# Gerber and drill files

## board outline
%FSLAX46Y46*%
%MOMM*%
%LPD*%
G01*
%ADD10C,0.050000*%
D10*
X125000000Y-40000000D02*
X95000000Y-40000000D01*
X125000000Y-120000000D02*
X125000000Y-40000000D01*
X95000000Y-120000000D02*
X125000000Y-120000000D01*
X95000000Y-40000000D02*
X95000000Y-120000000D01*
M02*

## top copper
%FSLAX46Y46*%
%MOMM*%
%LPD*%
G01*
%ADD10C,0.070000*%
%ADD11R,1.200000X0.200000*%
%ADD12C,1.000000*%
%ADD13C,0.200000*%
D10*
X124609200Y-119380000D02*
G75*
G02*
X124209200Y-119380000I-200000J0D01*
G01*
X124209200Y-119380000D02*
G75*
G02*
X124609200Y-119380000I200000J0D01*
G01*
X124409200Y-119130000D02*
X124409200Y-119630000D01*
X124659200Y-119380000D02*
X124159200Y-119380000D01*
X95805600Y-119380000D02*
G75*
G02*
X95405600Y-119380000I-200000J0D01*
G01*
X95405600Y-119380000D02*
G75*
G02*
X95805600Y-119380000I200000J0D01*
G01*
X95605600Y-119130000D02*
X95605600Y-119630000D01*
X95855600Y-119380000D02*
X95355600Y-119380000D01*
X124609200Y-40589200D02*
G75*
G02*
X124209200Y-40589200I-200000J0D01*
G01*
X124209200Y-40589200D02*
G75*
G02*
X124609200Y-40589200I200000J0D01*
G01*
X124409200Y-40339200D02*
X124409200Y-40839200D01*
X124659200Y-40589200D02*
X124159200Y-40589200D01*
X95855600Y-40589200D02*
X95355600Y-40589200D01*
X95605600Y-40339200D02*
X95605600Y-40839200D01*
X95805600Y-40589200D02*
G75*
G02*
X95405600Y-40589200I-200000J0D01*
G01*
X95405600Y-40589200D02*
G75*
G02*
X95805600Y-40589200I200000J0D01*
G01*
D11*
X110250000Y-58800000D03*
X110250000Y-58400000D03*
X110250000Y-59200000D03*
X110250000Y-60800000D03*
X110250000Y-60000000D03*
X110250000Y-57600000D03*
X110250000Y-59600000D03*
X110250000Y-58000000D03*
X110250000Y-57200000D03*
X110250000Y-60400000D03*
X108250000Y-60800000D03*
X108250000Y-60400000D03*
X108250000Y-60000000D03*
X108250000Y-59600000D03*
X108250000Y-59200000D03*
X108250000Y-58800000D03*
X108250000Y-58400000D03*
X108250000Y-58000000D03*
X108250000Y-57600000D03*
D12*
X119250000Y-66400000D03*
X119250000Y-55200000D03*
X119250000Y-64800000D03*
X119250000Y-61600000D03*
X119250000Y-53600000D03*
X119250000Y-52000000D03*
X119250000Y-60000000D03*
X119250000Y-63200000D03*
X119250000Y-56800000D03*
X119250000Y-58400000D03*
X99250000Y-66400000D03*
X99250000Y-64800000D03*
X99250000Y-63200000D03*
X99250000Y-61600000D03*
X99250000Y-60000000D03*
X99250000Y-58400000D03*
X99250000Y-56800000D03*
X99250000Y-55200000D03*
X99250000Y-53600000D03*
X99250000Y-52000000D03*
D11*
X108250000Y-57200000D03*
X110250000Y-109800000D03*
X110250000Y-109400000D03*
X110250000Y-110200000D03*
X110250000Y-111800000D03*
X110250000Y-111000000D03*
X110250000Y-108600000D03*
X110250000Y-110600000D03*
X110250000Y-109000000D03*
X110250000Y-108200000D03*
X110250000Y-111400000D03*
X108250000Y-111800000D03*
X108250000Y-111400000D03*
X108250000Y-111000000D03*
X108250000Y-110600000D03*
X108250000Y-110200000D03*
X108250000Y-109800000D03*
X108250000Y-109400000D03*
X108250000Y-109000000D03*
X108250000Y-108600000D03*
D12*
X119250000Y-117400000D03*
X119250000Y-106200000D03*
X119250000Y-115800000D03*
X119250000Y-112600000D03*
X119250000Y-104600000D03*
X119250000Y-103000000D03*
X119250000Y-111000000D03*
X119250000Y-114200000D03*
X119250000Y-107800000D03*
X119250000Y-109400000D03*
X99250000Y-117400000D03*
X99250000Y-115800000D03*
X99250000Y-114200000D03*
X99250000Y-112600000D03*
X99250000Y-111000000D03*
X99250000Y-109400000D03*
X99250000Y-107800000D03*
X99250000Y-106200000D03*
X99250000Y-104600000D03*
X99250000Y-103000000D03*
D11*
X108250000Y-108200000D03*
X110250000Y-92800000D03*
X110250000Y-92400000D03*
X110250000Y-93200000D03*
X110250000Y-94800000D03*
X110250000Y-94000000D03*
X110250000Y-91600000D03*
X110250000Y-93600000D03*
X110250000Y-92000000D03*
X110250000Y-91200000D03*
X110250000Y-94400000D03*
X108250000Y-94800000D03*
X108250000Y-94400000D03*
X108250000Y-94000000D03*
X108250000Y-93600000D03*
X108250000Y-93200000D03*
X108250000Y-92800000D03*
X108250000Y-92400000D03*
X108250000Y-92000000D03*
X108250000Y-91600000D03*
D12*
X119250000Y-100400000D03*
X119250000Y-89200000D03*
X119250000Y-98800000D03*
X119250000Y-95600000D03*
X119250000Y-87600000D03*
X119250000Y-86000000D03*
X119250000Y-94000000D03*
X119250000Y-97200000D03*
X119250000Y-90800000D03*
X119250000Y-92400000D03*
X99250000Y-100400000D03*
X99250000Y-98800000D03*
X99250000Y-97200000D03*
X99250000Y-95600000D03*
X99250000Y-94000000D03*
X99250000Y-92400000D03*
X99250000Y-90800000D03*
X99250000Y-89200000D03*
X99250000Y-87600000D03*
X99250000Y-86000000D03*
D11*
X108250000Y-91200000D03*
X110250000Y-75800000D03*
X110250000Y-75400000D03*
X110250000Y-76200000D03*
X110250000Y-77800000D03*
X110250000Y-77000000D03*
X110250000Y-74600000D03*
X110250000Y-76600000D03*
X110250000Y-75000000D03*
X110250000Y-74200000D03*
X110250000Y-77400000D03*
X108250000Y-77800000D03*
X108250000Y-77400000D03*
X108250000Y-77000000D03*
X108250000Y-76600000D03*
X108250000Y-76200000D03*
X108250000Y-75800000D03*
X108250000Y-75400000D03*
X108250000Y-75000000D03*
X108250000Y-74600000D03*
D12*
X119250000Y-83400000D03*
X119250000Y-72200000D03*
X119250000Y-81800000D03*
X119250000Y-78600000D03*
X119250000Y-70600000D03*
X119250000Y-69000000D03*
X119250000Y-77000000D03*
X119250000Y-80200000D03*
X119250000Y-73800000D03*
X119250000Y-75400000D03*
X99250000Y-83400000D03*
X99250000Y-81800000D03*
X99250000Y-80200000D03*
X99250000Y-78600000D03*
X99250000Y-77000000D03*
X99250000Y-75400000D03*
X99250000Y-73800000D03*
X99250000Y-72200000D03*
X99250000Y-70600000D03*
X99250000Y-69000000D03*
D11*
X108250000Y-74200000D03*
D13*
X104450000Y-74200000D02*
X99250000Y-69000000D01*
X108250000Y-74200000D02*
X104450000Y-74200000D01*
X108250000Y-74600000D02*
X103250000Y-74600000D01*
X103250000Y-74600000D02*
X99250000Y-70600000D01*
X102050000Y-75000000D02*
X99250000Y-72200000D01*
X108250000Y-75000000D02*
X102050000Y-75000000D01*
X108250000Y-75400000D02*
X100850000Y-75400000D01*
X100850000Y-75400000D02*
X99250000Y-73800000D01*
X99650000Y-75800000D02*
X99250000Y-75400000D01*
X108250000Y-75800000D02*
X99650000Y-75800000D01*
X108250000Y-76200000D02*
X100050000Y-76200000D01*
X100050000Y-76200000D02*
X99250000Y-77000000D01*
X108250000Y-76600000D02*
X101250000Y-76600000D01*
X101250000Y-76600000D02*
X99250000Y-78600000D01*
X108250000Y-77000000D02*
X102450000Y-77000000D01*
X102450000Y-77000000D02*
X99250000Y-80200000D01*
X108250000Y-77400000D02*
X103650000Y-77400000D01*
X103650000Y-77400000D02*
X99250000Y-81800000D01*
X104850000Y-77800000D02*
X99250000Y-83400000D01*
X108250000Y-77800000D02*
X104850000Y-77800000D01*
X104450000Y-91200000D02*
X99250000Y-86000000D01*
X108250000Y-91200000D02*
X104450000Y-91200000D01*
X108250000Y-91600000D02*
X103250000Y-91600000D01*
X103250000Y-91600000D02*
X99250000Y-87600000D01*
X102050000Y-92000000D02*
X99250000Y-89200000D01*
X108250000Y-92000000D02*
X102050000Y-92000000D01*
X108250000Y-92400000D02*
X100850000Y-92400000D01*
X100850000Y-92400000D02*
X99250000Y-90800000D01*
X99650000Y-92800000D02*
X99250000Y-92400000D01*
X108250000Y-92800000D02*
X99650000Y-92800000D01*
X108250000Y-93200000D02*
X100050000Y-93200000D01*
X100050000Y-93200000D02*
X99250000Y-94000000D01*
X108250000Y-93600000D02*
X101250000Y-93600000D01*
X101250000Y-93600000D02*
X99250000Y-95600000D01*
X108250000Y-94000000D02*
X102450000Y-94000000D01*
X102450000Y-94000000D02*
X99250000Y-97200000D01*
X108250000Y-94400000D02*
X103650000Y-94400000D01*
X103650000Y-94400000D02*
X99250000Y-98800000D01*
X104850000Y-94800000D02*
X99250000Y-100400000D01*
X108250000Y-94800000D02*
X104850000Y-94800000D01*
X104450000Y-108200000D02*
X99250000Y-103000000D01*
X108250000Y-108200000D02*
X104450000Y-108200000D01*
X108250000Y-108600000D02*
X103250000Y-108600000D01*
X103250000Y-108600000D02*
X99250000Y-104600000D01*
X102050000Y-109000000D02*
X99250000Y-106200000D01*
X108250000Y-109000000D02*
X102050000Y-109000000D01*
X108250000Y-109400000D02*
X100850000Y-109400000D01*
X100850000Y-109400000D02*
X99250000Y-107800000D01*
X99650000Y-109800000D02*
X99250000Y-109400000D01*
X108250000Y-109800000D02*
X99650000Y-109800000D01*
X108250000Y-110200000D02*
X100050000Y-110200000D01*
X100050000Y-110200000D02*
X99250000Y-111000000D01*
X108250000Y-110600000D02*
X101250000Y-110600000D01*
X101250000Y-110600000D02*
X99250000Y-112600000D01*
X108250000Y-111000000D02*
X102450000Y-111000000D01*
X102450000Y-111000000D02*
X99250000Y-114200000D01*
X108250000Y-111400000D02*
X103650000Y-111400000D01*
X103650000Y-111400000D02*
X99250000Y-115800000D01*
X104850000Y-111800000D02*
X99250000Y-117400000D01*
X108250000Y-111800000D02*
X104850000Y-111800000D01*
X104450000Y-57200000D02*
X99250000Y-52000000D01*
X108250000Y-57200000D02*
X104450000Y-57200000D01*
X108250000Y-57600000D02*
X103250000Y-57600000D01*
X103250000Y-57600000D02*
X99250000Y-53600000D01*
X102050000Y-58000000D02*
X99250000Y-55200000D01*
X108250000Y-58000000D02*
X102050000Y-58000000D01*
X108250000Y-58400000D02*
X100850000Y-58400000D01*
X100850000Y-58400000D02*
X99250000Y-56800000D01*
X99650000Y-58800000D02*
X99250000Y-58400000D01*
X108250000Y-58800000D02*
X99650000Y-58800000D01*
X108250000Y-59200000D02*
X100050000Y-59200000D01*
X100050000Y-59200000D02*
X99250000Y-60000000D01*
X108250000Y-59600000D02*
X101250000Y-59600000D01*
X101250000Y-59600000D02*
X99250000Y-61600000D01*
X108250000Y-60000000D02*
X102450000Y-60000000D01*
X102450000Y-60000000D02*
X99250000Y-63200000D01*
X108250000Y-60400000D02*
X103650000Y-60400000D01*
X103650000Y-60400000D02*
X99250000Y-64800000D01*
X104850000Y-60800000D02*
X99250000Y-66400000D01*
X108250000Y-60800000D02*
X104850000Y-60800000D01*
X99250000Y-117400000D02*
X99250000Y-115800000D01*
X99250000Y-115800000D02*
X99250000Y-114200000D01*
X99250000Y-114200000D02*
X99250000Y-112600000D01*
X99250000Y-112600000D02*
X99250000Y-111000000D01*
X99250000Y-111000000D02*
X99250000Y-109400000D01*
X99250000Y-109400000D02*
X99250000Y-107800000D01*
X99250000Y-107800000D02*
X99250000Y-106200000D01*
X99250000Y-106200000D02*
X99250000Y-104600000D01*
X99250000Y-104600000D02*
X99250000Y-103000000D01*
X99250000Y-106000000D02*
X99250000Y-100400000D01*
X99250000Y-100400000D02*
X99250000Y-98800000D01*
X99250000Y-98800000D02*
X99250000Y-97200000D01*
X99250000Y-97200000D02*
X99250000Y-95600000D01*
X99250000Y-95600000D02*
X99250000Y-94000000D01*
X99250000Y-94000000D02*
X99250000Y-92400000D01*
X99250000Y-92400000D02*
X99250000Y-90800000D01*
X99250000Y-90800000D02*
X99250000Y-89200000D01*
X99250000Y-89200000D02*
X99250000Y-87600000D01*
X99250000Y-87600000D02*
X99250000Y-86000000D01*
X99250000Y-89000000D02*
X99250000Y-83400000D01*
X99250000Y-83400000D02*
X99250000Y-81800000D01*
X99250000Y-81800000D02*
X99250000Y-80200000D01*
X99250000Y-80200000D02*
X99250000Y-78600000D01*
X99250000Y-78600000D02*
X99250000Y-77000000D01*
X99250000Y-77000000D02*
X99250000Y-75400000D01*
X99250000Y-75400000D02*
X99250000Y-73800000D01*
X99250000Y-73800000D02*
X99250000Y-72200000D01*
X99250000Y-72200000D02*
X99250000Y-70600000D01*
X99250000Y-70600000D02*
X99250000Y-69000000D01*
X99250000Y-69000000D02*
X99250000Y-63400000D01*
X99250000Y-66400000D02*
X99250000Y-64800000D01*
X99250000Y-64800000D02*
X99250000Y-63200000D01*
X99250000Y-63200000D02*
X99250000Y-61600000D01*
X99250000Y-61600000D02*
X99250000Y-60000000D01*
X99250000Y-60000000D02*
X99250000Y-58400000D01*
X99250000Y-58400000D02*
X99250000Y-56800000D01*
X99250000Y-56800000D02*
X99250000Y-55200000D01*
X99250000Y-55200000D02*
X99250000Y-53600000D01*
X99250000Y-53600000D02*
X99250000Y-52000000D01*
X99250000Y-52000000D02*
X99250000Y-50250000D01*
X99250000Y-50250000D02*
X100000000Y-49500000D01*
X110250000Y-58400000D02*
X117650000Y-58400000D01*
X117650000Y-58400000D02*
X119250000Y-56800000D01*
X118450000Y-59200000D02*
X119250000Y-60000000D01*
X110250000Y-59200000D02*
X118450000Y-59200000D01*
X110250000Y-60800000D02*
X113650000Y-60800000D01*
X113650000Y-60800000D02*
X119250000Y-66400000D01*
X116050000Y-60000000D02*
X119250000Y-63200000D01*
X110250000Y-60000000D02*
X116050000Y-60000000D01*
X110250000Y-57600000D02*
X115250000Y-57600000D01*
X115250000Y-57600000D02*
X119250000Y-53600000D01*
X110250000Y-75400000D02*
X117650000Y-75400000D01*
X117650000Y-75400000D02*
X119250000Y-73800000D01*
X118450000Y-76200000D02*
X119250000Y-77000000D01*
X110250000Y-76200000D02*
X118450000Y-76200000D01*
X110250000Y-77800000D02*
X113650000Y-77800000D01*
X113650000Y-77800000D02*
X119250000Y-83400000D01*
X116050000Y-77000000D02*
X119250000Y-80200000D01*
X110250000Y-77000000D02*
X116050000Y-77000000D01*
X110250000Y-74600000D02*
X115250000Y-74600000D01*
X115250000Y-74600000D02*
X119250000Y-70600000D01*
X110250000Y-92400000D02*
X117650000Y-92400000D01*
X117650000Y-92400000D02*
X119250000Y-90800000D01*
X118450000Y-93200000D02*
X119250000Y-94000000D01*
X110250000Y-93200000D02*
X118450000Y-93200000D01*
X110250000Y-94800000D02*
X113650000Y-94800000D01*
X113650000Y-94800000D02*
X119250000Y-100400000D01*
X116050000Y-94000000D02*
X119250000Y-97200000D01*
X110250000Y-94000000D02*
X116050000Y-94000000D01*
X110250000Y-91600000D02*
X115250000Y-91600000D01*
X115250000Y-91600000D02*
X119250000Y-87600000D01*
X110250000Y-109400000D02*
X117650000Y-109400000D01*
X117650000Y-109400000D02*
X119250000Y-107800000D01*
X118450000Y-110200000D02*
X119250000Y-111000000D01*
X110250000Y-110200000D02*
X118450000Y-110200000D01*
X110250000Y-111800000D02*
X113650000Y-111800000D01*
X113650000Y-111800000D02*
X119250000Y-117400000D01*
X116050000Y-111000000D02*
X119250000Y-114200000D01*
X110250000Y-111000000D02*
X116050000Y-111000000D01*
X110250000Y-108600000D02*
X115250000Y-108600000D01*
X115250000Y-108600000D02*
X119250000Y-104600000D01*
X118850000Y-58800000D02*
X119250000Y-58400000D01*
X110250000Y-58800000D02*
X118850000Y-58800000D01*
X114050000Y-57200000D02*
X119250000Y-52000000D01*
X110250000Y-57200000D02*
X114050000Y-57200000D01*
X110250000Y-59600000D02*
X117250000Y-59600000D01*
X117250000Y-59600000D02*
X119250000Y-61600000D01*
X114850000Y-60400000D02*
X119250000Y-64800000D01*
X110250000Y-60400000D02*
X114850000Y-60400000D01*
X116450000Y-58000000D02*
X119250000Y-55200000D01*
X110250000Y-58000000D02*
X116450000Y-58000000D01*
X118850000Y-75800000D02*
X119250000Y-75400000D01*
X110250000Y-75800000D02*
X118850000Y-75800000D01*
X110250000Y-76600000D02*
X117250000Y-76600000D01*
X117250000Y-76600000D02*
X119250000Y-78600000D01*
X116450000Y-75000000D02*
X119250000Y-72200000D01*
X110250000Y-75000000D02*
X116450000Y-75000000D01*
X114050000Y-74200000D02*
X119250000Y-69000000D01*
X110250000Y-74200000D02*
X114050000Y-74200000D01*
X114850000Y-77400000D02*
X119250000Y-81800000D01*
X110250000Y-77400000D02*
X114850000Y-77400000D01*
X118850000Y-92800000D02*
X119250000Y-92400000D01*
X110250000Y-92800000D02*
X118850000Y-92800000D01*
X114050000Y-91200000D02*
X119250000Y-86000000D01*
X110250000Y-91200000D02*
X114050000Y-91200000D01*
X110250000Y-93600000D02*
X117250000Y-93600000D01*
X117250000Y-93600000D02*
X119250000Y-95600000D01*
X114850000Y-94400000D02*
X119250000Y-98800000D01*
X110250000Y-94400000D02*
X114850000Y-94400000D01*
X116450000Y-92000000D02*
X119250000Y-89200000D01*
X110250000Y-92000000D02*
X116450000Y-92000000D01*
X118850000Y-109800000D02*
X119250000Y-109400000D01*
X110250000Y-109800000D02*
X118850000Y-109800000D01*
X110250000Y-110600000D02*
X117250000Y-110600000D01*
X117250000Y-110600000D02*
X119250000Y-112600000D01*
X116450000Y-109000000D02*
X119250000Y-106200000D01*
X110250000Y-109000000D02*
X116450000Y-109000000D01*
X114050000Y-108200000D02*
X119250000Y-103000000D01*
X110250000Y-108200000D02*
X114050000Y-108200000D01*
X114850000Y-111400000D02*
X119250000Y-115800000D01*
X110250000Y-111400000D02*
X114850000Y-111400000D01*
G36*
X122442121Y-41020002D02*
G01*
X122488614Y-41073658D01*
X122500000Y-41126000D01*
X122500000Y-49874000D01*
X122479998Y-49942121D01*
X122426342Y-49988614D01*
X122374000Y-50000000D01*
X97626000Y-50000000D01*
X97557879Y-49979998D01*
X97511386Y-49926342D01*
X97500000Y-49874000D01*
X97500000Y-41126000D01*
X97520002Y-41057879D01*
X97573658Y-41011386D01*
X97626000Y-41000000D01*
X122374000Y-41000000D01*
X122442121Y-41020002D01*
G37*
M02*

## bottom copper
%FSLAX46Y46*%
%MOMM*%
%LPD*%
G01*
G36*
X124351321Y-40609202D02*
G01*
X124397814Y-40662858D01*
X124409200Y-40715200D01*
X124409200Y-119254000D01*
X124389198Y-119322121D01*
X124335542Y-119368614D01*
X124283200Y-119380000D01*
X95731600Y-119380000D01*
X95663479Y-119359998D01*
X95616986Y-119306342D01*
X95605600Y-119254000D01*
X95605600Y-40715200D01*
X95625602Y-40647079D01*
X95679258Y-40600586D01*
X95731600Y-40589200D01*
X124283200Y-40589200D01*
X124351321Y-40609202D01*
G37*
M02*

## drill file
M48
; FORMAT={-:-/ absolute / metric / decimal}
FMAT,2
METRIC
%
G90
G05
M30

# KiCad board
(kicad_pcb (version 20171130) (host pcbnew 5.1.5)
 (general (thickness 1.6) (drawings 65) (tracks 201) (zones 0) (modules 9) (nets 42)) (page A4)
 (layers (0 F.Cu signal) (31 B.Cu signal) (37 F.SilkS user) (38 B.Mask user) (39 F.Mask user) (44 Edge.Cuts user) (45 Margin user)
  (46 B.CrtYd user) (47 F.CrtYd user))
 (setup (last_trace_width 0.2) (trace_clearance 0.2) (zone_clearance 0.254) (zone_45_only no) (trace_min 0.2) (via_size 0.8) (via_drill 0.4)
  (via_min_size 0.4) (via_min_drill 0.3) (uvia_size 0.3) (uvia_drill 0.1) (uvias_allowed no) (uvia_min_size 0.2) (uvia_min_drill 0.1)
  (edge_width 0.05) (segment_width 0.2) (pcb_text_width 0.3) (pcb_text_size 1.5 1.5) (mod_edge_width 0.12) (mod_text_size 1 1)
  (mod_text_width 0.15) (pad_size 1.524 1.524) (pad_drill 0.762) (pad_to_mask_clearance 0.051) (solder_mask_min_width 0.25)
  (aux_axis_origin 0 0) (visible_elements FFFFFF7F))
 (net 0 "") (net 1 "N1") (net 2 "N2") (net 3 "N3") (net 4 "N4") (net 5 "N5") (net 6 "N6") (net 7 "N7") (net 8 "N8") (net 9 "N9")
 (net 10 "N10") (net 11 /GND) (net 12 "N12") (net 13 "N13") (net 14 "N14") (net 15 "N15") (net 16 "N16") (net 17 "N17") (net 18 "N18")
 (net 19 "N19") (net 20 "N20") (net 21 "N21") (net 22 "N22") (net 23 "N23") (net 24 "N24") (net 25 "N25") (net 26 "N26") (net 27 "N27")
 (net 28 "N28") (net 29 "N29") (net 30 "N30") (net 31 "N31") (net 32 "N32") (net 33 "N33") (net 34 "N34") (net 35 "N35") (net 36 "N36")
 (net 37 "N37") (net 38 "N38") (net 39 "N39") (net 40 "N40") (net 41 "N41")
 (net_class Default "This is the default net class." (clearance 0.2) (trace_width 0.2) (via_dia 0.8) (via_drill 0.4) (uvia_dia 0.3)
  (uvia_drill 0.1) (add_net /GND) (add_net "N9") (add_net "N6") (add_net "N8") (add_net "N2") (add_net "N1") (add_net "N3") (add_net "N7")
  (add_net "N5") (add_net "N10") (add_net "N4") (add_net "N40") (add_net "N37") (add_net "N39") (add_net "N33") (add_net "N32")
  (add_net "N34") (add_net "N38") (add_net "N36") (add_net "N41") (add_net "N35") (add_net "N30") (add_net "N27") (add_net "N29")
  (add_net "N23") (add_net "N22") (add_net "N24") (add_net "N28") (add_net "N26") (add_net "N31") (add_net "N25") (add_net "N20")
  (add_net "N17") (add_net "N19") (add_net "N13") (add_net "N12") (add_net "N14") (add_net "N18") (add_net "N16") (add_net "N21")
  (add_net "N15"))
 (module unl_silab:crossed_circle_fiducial (layer F.Cu) (at 124.4092 119.38)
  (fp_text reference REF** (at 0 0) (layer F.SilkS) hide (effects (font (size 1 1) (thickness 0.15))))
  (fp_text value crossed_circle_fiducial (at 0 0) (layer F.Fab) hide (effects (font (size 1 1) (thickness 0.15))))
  (fp_circle (center 0 0) (end 0.2 0) (layer F.Cu) (width 0.07))
  (fp_line (start 0 -0.25) (end 0 0.25) (layer F.Cu) (width 0.07))
  (fp_line (start 0.25 0) (end -0.25 0) (layer F.Cu) (width 0.07)))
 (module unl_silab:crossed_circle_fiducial (layer F.Cu) (at 95.6056 119.38)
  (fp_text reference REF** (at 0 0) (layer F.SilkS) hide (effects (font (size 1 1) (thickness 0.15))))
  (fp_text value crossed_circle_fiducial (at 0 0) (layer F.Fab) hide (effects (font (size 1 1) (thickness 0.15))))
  (fp_circle (center 0 0) (end 0.2 0) (layer F.Cu) (width 0.07))
  (fp_line (start 0 -0.25) (end 0 0.25) (layer F.Cu) (width 0.07))
  (fp_line (start 0.25 0) (end -0.25 0) (layer F.Cu) (width 0.07)))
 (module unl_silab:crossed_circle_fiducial (layer F.Cu) (at 124.4092 40.5892)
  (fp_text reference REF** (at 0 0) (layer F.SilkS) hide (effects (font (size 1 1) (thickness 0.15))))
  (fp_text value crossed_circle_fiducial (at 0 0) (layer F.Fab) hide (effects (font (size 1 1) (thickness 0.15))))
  (fp_circle (center 0 0) (end 0.2 0) (layer F.Cu) (width 0.07))
  (fp_line (start 0 -0.25) (end 0 0.25) (layer F.Cu) (width 0.07))
  (fp_line (start 0.25 0) (end -0.25 0) (layer F.Cu) (width 0.07)))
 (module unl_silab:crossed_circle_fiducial (layer F.Cu) (at 95.6056 40.5892)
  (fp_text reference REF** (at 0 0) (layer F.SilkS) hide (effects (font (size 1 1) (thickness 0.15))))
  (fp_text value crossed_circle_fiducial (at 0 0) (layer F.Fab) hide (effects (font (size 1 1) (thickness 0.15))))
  (fp_line (start 0.25 0) (end -0.25 0) (layer F.Cu) (width 0.07))
  (fp_line (start 0 -0.25) (end 0 0.25) (layer F.Cu) (width 0.07))
  (fp_circle (center 0 0) (end 0.2 0) (layer F.Cu) (width 0.07)))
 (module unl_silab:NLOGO (layer F.Cu) (at 108.75 115.25)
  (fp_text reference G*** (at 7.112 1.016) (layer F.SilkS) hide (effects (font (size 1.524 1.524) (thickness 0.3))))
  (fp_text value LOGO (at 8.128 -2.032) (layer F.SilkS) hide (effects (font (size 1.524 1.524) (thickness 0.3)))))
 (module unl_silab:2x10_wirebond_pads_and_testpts (layer F.Cu) (at 109.25 59)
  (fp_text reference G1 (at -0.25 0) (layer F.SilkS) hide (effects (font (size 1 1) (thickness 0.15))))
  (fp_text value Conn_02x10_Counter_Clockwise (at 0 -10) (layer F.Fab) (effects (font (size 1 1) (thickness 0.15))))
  (pad 15 smd rect (at 1 -0.2) (size 1.2 0.2) (layers F.Cu F.Paste F.Mask) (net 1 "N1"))
  (pad 14 smd rect (at 1 -0.6) (size 1.2 0.2) (layers F.Cu F.Paste F.Mask) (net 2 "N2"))
  (pad 16 smd rect (at 1 0.2) (size 1.2 0.2) (layers F.Cu F.Paste F.Mask) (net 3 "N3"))
  (pad 20 smd rect (at 1 1.8) (size 1.2 0.2) (layers F.Cu F.Paste F.Mask) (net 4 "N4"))
  (pad 18 smd rect (at 1 1) (size 1.2 0.2) (layers F.Cu F.Paste F.Mask) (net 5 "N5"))
  (pad 12 smd rect (at 1 -1.4) (size 1.2 0.2) (layers F.Cu F.Paste F.Mask) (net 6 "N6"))
  (pad 17 smd rect (at 1 0.6) (size 1.2 0.2) (layers F.Cu F.Paste F.Mask) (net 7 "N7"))
  (pad 13 smd rect (at 1 -1) (size 1.2 0.2) (layers F.Cu F.Paste F.Mask) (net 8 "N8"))
  (pad 11 smd rect (at 1 -1.8) (size 1.2 0.2) (layers F.Cu F.Paste F.Mask) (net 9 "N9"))
  (pad 19 smd rect (at 1 1.4) (size 1.2 0.2) (layers F.Cu F.Paste F.Mask) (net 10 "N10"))
  (pad 10 smd rect (at -1 1.8) (size 1.2 0.2) (layers F.Cu F.Paste F.Mask) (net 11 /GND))
  (pad 9 smd rect (at -1 1.4) (size 1.2 0.2) (layers F.Cu F.Paste F.Mask) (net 11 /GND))
  (pad 8 smd rect (at -1 1) (size 1.2 0.2) (layers F.Cu F.Paste F.Mask) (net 11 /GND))
  (pad 7 smd rect (at -1 0.6) (size 1.2 0.2) (layers F.Cu F.Paste F.Mask) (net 11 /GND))
  (pad 6 smd rect (at -1 0.2) (size 1.2 0.2) (layers F.Cu F.Paste F.Mask) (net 11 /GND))
  (pad 5 smd rect (at -1 -0.2) (size 1.2 0.2) (layers F.Cu F.Paste F.Mask) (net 11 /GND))
  (pad 4 smd rect (at -1 -0.6) (size 1.2 0.2) (layers F.Cu F.Paste F.Mask) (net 11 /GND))
  (pad 3 smd rect (at -1 -1) (size 1.2 0.2) (layers F.Cu F.Paste F.Mask) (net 11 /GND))
  (pad 2 smd rect (at -1 -1.4) (size 1.2 0.2) (layers F.Cu F.Paste F.Mask) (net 11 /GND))
  (pad 20 smd circle (at 10 7.4) (size 1 1) (layers F.Cu F.Paste F.Mask) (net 4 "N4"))
  (pad 13 smd circle (at 10 -3.8) (size 1 1) (layers F.Cu F.Paste F.Mask) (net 8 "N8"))
  (pad 19 smd circle (at 10 5.8) (size 1 1) (layers F.Cu F.Paste F.Mask) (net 10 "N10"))
  (pad 17 smd circle (at 10 2.6) (size 1 1) (layers F.Cu F.Paste F.Mask) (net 7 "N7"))
  (pad 12 smd circle (at 10 -5.4) (size 1 1) (layers F.Cu F.Paste F.Mask) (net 6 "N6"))
  (pad 11 smd circle (at 10 -7) (size 1 1) (layers F.Cu F.Paste F.Mask) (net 9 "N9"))
  (pad 16 smd circle (at 10 1) (size 1 1) (layers F.Cu F.Paste F.Mask) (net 3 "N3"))
  (pad 18 smd circle (at 10 4.2) (size 1 1) (layers F.Cu F.Paste F.Mask) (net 5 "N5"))
  (pad 14 smd circle (at 10 -2.2) (size 1 1) (layers F.Cu F.Paste F.Mask) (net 2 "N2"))
  (pad 15 smd circle (at 10 -0.6) (size 1 1) (layers F.Cu F.Paste F.Mask) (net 1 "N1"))
  (pad 10 smd circle (at -10 7.4) (size 1 1) (layers F.Cu F.Paste F.Mask) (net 11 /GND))
  (pad 9 smd circle (at -10 5.8) (size 1 1) (layers F.Cu F.Paste F.Mask) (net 11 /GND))
  (pad 8 smd circle (at -10 4.2) (size 1 1) (layers F.Cu F.Paste F.Mask) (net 11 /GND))
  (pad 7 smd circle (at -10 2.6) (size 1 1) (layers F.Cu F.Paste F.Mask) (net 11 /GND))
  (pad 6 smd circle (at -10 1) (size 1 1) (layers F.Cu F.Paste F.Mask) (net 11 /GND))
  (pad 5 smd circle (at -10 -0.6) (size 1 1) (layers F.Cu F.Paste F.Mask) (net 11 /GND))
  (pad 4 smd circle (at -10 -2.2) (size 1 1) (layers F.Cu F.Paste F.Mask) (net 11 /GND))
  (pad 3 smd circle (at -10 -3.8) (size 1 1) (layers F.Cu F.Paste F.Mask) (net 11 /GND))
  (pad 2 smd circle (at -10 -5.4) (size 1 1) (layers F.Cu F.Paste F.Mask) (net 11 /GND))
  (pad 1 smd circle (at -10 -7) (size 1 1) (layers F.Cu F.Paste F.Mask) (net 11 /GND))
  (pad 1 smd rect (at -1 -1.8) (size 1.2 0.2) (layers F.Cu F.Paste F.Mask) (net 11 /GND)))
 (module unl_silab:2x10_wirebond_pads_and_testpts (layer F.Cu) (at 109.25 110)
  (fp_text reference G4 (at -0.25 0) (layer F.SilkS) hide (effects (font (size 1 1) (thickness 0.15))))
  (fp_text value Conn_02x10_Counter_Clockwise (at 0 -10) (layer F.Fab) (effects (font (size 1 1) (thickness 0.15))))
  (pad 15 smd rect (at 1 -0.2) (size 1.2 0.2) (layers F.Cu F.Paste F.Mask) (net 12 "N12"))
  (pad 14 smd rect (at 1 -0.6) (size 1.2 0.2) (layers F.Cu F.Paste F.Mask) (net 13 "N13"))
  (pad 16 smd rect (at 1 0.2) (size 1.2 0.2) (layers F.Cu F.Paste F.Mask) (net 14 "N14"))
  (pad 20 smd rect (at 1 1.8) (size 1.2 0.2) (layers F.Cu F.Paste F.Mask) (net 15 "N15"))
  (pad 18 smd rect (at 1 1) (size 1.2 0.2) (layers F.Cu F.Paste F.Mask) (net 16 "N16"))
  (pad 12 smd rect (at 1 -1.4) (size 1.2 0.2) (layers F.Cu F.Paste F.Mask) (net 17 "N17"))
  (pad 17 smd rect (at 1 0.6) (size 1.2 0.2) (layers F.Cu F.Paste F.Mask) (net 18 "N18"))
  (pad 13 smd rect (at 1 -1) (size 1.2 0.2) (layers F.Cu F.Paste F.Mask) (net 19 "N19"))
  (pad 11 smd rect (at 1 -1.8) (size 1.2 0.2) (layers F.Cu F.Paste F.Mask) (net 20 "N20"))
  (pad 19 smd rect (at 1 1.4) (size 1.2 0.2) (layers F.Cu F.Paste F.Mask) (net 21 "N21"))
  (pad 10 smd rect (at -1 1.8) (size 1.2 0.2) (layers F.Cu F.Paste F.Mask) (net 11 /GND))
  (pad 9 smd rect (at -1 1.4) (size 1.2 0.2) (layers F.Cu F.Paste F.Mask) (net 11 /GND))
  (pad 8 smd rect (at -1 1) (size 1.2 0.2) (layers F.Cu F.Paste F.Mask) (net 11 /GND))
  (pad 7 smd rect (at -1 0.6) (size 1.2 0.2) (layers F.Cu F.Paste F.Mask) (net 11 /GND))
  (pad 6 smd rect (at -1 0.2) (size 1.2 0.2) (layers F.Cu F.Paste F.Mask) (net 11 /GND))
  (pad 5 smd rect (at -1 -0.2) (size 1.2 0.2) (layers F.Cu F.Paste F.Mask) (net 11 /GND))
  (pad 4 smd rect (at -1 -0.6) (size 1.2 0.2) (layers F.Cu F.Paste F.Mask) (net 11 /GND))
  (pad 3 smd rect (at -1 -1) (size 1.2 0.2) (layers F.Cu F.Paste F.Mask) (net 11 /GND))
  (pad 2 smd rect (at -1 -1.4) (size 1.2 0.2) (layers F.Cu F.Paste F.Mask) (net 11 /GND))
  (pad 20 smd circle (at 10 7.4) (size 1 1) (layers F.Cu F.Paste F.Mask) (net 15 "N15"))
  (pad 13 smd circle (at 10 -3.8) (size 1 1) (layers F.Cu F.Paste F.Mask) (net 19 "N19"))
  (pad 19 smd circle (at 10 5.8) (size 1 1) (layers F.Cu F.Paste F.Mask) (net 21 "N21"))
  (pad 17 smd circle (at 10 2.6) (size 1 1) (layers F.Cu F.Paste F.Mask) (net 18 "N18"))
  (pad 12 smd circle (at 10 -5.4) (size 1 1) (layers F.Cu F.Paste F.Mask) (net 17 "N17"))
  (pad 11 smd circle (at 10 -7) (size 1 1) (layers F.Cu F.Paste F.Mask) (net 20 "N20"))
  (pad 16 smd circle (at 10 1) (size 1 1) (layers F.Cu F.Paste F.Mask) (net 14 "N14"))
  (pad 18 smd circle (at 10 4.2) (size 1 1) (layers F.Cu F.Paste F.Mask) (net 16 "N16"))
  (pad 14 smd circle (at 10 -2.2) (size 1 1) (layers F.Cu F.Paste F.Mask) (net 13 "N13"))
  (pad 15 smd circle (at 10 -0.6) (size 1 1) (layers F.Cu F.Paste F.Mask) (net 12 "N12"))
  (pad 10 smd circle (at -10 7.4) (size 1 1) (layers F.Cu F.Paste F.Mask) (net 11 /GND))
  (pad 9 smd circle (at -10 5.8) (size 1 1) (layers F.Cu F.Paste F.Mask) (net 11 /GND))
  (pad 8 smd circle (at -10 4.2) (size 1 1) (layers F.Cu F.Paste F.Mask) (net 11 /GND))
  (pad 7 smd circle (at -10 2.6) (size 1 1) (layers F.Cu F.Paste F.Mask) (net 11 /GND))
  (pad 6 smd circle (at -10 1) (size 1 1) (layers F.Cu F.Paste F.Mask) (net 11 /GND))
  (pad 5 smd circle (at -10 -0.6) (size 1 1) (layers F.Cu F.Paste F.Mask) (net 11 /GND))
  (pad 4 smd circle (at -10 -2.2) (size 1 1) (layers F.Cu F.Paste F.Mask) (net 11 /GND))
  (pad 3 smd circle (at -10 -3.8) (size 1 1) (layers F.Cu F.Paste F.Mask) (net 11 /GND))
  (pad 2 smd circle (at -10 -5.4) (size 1 1) (layers F.Cu F.Paste F.Mask) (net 11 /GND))
  (pad 1 smd circle (at -10 -7) (size 1 1) (layers F.Cu F.Paste F.Mask) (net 11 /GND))
  (pad 1 smd rect (at -1 -1.8) (size 1.2 0.2) (layers F.Cu F.Paste F.Mask) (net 11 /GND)))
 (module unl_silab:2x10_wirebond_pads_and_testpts (layer F.Cu) (at 109.25 93)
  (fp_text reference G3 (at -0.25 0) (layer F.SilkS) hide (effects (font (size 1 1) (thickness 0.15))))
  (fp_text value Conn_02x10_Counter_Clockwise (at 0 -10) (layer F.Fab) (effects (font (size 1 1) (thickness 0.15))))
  (pad 15 smd rect (at 1 -0.2) (size 1.2 0.2) (layers F.Cu F.Paste F.Mask) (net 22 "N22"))
  (pad 14 smd rect (at 1 -0.6) (size 1.2 0.2) (layers F.Cu F.Paste F.Mask) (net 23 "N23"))
  (pad 16 smd rect (at 1 0.2) (size 1.2 0.2) (layers F.Cu F.Paste F.Mask) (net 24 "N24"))
  (pad 20 smd rect (at 1 1.8) (size 1.2 0.2) (layers F.Cu F.Paste F.Mask) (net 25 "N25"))
  (pad 18 smd rect (at 1 1) (size 1.2 0.2) (layers F.Cu F.Paste F.Mask) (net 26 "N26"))
  (pad 12 smd rect (at 1 -1.4) (size 1.2 0.2) (layers F.Cu F.Paste F.Mask) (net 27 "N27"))
  (pad 17 smd rect (at 1 0.6) (size 1.2 0.2) (layers F.Cu F.Paste F.Mask) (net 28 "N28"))
  (pad 13 smd rect (at 1 -1) (size 1.2 0.2) (layers F.Cu F.Paste F.Mask) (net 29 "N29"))
  (pad 11 smd rect (at 1 -1.8) (size 1.2 0.2) (layers F.Cu F.Paste F.Mask) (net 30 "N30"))
  (pad 19 smd rect (at 1 1.4) (size 1.2 0.2) (layers F.Cu F.Paste F.Mask) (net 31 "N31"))
  (pad 10 smd rect (at -1 1.8) (size 1.2 0.2) (layers F.Cu F.Paste F.Mask) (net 11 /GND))
  (pad 9 smd rect (at -1 1.4) (size 1.2 0.2) (layers F.Cu F.Paste F.Mask) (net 11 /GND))
  (pad 8 smd rect (at -1 1) (size 1.2 0.2) (layers F.Cu F.Paste F.Mask) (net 11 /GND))
  (pad 7 smd rect (at -1 0.6) (size 1.2 0.2) (layers F.Cu F.Paste F.Mask) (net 11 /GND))
  (pad 6 smd rect (at -1 0.2) (size 1.2 0.2) (layers F.Cu F.Paste F.Mask) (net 11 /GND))
  (pad 5 smd rect (at -1 -0.2) (size 1.2 0.2) (layers F.Cu F.Paste F.Mask) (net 11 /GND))
  (pad 4 smd rect (at -1 -0.6) (size 1.2 0.2) (layers F.Cu F.Paste F.Mask) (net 11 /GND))
  (pad 3 smd rect (at -1 -1) (size 1.2 0.2) (layers F.Cu F.Paste F.Mask) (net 11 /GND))
  (pad 2 smd rect (at -1 -1.4) (size 1.2 0.2) (layers F.Cu F.Paste F.Mask) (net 11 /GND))
  (pad 20 smd circle (at 10 7.4) (size 1 1) (layers F.Cu F.Paste F.Mask) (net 25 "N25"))
  (pad 13 smd circle (at 10 -3.8) (size 1 1) (layers F.Cu F.Paste F.Mask) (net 29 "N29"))
  (pad 19 smd circle (at 10 5.8) (size 1 1) (layers F.Cu F.Paste F.Mask) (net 31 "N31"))
  (pad 17 smd circle (at 10 2.6) (size 1 1) (layers F.Cu F.Paste F.Mask) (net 28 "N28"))
  (pad 12 smd circle (at 10 -5.4) (size 1 1) (layers F.Cu F.Paste F.Mask) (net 27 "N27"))
  (pad 11 smd circle (at 10 -7) (size 1 1) (layers F.Cu F.Paste F.Mask) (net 30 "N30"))
  (pad 16 smd circle (at 10 1) (size 1 1) (layers F.Cu F.Paste F.Mask) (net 24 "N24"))
  (pad 18 smd circle (at 10 4.2) (size 1 1) (layers F.Cu F.Paste F.Mask) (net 26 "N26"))
  (pad 14 smd circle (at 10 -2.2) (size 1 1) (layers F.Cu F.Paste F.Mask) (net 23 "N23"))
  (pad 15 smd circle (at 10 -0.6) (size 1 1) (layers F.Cu F.Paste F.Mask) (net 22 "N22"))
  (pad 10 smd circle (at -10 7.4) (size 1 1) (layers F.Cu F.Paste F.Mask) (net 11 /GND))
  (pad 9 smd circle (at -10 5.8) (size 1 1) (layers F.Cu F.Paste F.Mask) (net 11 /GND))
  (pad 8 smd circle (at -10 4.2) (size 1 1) (layers F.Cu F.Paste F.Mask) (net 11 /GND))
  (pad 7 smd circle (at -10 2.6) (size 1 1) (layers F.Cu F.Paste F.Mask) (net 11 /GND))
  (pad 6 smd circle (at -10 1) (size 1 1) (layers F.Cu F.Paste F.Mask) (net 11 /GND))
  (pad 5 smd circle (at -10 -0.6) (size 1 1) (layers F.Cu F.Paste F.Mask) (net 11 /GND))
  (pad 4 smd circle (at -10 -2.2) (size 1 1) (layers F.Cu F.Paste F.Mask) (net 11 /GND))
  (pad 3 smd circle (at -10 -3.8) (size 1 1) (layers F.Cu F.Paste F.Mask) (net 11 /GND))
  (pad 2 smd circle (at -10 -5.4) (size 1 1) (layers F.Cu F.Paste F.Mask) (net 11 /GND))
  (pad 1 smd circle (at -10 -7) (size 1 1) (layers F.Cu F.Paste F.Mask) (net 11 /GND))
  (pad 1 smd rect (at -1 -1.8) (size 1.2 0.2) (layers F.Cu F.Paste F.Mask) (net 11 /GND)))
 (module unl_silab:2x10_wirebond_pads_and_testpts (layer F.Cu) (at 109.25 76)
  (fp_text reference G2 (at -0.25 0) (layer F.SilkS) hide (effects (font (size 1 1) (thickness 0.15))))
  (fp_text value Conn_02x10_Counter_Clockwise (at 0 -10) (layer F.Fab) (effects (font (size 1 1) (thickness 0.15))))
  (pad 15 smd rect (at 1 -0.2) (size 1.2 0.2) (layers F.Cu F.Paste F.Mask) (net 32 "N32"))
  (pad 14 smd rect (at 1 -0.6) (size 1.2 0.2) (layers F.Cu F.Paste F.Mask) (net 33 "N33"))
  (pad 16 smd rect (at 1 0.2) (size 1.2 0.2) (layers F.Cu F.Paste F.Mask) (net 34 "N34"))
  (pad 20 smd rect (at 1 1.8) (size 1.2 0.2) (layers F.Cu F.Paste F.Mask) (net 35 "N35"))
  (pad 18 smd rect (at 1 1) (size 1.2 0.2) (layers F.Cu F.Paste F.Mask) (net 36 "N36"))
  (pad 12 smd rect (at 1 -1.4) (size 1.2 0.2) (layers F.Cu F.Paste F.Mask) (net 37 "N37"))
  (pad 17 smd rect (at 1 0.6) (size 1.2 0.2) (layers F.Cu F.Paste F.Mask) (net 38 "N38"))
  (pad 13 smd rect (at 1 -1) (size 1.2 0.2) (layers F.Cu F.Paste F.Mask) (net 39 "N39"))
  (pad 11 smd rect (at 1 -1.8) (size 1.2 0.2) (layers F.Cu F.Paste F.Mask) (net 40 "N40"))
  (pad 19 smd rect (at 1 1.4) (size 1.2 0.2) (layers F.Cu F.Paste F.Mask) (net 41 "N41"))
  (pad 10 smd rect (at -1 1.8) (size 1.2 0.2) (layers F.Cu F.Paste F.Mask) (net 11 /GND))
  (pad 9 smd rect (at -1 1.4) (size 1.2 0.2) (layers F.Cu F.Paste F.Mask) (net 11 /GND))
  (pad 8 smd rect (at -1 1) (size 1.2 0.2) (layers F.Cu F.Paste F.Mask) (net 11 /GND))
  (pad 7 smd rect (at -1 0.6) (size 1.2 0.2) (layers F.Cu F.Paste F.Mask) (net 11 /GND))
  (pad 6 smd rect (at -1 0.2) (size 1.2 0.2) (layers F.Cu F.Paste F.Mask) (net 11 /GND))
  (pad 5 smd rect (at -1 -0.2) (size 1.2 0.2) (layers F.Cu F.Paste F.Mask) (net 11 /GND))
  (pad 4 smd rect (at -1 -0.6) (size 1.2 0.2) (layers F.Cu F.Paste F.Mask) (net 11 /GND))
  (pad 3 smd rect (at -1 -1) (size 1.2 0.2) (layers F.Cu F.Paste F.Mask) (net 11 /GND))
  (pad 2 smd rect (at -1 -1.4) (size 1.2 0.2) (layers F.Cu F.Paste F.Mask) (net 11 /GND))
  (pad 20 smd circle (at 10 7.4) (size 1 1) (layers F.Cu F.Paste F.Mask) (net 35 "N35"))
  (pad 13 smd circle (at 10 -3.8) (size 1 1) (layers F.Cu F.Paste F.Mask) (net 39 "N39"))
  (pad 19 smd circle (at 10 5.8) (size 1 1) (layers F.Cu F.Paste F.Mask) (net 41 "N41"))
  (pad 17 smd circle (at 10 2.6) (size 1 1) (layers F.Cu F.Paste F.Mask) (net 38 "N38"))
  (pad 12 smd circle (at 10 -5.4) (size 1 1) (layers F.Cu F.Paste F.Mask) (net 37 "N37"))
  (pad 11 smd circle (at 10 -7) (size 1 1) (layers F.Cu F.Paste F.Mask) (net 40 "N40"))
  (pad 16 smd circle (at 10 1) (size 1 1) (layers F.Cu F.Paste F.Mask) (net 34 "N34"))
  (pad 18 smd circle (at 10 4.2) (size 1 1) (layers F.Cu F.Paste F.Mask) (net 36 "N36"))
  (pad 14 smd circle (at 10 -2.2) (size 1 1) (layers F.Cu F.Paste F.Mask) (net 33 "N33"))
  (pad 15 smd circle (at 10 -0.6) (size 1 1) (layers F.Cu F.Paste F.Mask) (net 32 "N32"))
  (pad 10 smd circle (at -10 7.4) (size 1 1) (layers F.Cu F.Paste F.Mask) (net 11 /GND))
  (pad 9 smd circle (at -10 5.8) (size 1 1) (layers F.Cu F.Paste F.Mask) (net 11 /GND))
  (pad 8 smd circle (at -10 4.2) (size 1 1) (layers F.Cu F.Paste F.Mask) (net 11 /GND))
  (pad 7 smd circle (at -10 2.6) (size 1 1) (layers F.Cu F.Paste F.Mask) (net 11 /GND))
  (pad 6 smd circle (at -10 1) (size 1 1) (layers F.Cu F.Paste F.Mask) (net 11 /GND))
  (pad 5 smd circle (at -10 -0.6) (size 1 1) (layers F.Cu F.Paste F.Mask) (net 11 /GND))
  (pad 4 smd circle (at -10 -2.2) (size 1 1) (layers F.Cu F.Paste F.Mask) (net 11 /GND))
  (pad 3 smd circle (at -10 -3.8) (size 1 1) (layers F.Cu F.Paste F.Mask) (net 11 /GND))
  (pad 2 smd circle (at -10 -5.4) (size 1 1) (layers F.Cu F.Paste F.Mask) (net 11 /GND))
  (pad 1 smd circle (at -10 -7) (size 1 1) (layers F.Cu F.Paste F.Mask) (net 11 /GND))
  (pad 1 smd rect (at -1 -1.8) (size 1.2 0.2) (layers F.Cu F.Paste F.Mask) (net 11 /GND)))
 (gr_line (start 125 40) (end 95 40) (layer Edge.Cuts) (width 0.05))
 (gr_line (start 125 120) (end 125 40) (layer Edge.Cuts) (width 0.05))
 (gr_line (start 95 120) (end 125 120) (layer Edge.Cuts) (width 0.05))
 (gr_line (start 95 40) (end 95 120) (layer Edge.Cuts) (width 0.05))
 (segment (start 104.45 74.2) (end 99.25 69) (width 0.2) (layer F.Cu) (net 11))
 (segment (start 108.25 74.2) (end 104.45 74.2) (width 0.2) (layer F.Cu) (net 11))
 (segment (start 108.25 74.6) (end 103.25 74.6) (width 0.2) (layer F.Cu) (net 11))
 (segment (start 103.25 74.6) (end 99.25 70.6) (width 0.2) (layer F.Cu) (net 11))
 (segment (start 102.05 75) (end 99.25 72.2) (width 0.2) (layer F.Cu) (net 11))
 (segment (start 108.25 75) (end 102.05 75) (width 0.2) (layer F.Cu) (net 11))
 (segment (start 108.25 75.4) (end 100.85 75.4) (width 0.2) (layer F.Cu) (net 11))
 (segment (start 100.85 75.4) (end 99.25 73.8) (width 0.2) (layer F.Cu) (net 11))
 (segment (start 99.65 75.8) (end 99.25 75.4) (width 0.2) (layer F.Cu) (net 11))
 (segment (start 108.25 75.8) (end 99.65 75.8) (width 0.2) (layer F.Cu) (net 11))
 (segment (start 108.25 76.2) (end 100.05 76.2) (width 0.2) (layer F.Cu) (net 11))
 (segment (start 100.05 76.2) (end 99.25 77) (width 0.2) (layer F.Cu) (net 11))
 (segment (start 108.25 76.6) (end 101.25 76.6) (width 0.2) (layer F.Cu) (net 11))
 (segment (start 101.25 76.6) (end 99.25 78.6) (width 0.2) (layer F.Cu) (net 11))
 (segment (start 108.25 77) (end 102.45 77) (width 0.2) (layer F.Cu) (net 11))
 (segment (start 102.45 77) (end 99.25 80.2) (width 0.2) (layer F.Cu) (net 11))
 (segment (start 108.25 77.4) (end 103.65 77.4) (width 0.2) (layer F.Cu) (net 11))
 (segment (start 103.65 77.4) (end 99.25 81.8) (width 0.2) (layer F.Cu) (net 11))
 (segment (start 104.85 77.8) (end 99.25 83.4) (width 0.2) (layer F.Cu) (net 11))
 (segment (start 108.25 77.8) (end 104.85 77.8) (width 0.2) (layer F.Cu) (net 11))
 (segment (start 104.45 91.2) (end 99.25 86) (width 0.2) (layer F.Cu) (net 11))
 (segment (start 108.25 91.2) (end 104.45 91.2) (width 0.2) (layer F.Cu) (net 11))
 (segment (start 108.25 91.6) (end 103.25 91.6) (width 0.2) (layer F.Cu) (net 11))
 (segment (start 103.25 91.6) (end 99.25 87.6) (width 0.2) (layer F.Cu) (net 11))
 (segment (start 102.05 92) (end 99.25 89.2) (width 0.2) (layer F.Cu) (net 11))
 (segment (start 108.25 92) (end 102.05 92) (width 0.2) (layer F.Cu) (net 11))
 (segment (start 108.25 92.4) (end 100.85 92.4) (width 0.2) (layer F.Cu) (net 11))
 (segment (start 100.85 92.4) (end 99.25 90.8) (width 0.2) (layer F.Cu) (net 11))
 (segment (start 99.65 92.8) (end 99.25 92.4) (width 0.2) (layer F.Cu) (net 11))
 (segment (start 108.25 92.8) (end 99.65 92.8) (width 0.2) (layer F.Cu) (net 11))
 (segment (start 108.25 93.2) (end 100.05 93.2) (width 0.2) (layer F.Cu) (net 11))
 (segment (start 100.05 93.2) (end 99.25 94) (width 0.2) (layer F.Cu) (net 11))
 (segment (start 108.25 93.6) (end 101.25 93.6) (width 0.2) (layer F.Cu) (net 11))
 (segment (start 101.25 93.6) (end 99.25 95.6) (width 0.2) (layer F.Cu) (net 11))
 (segment (start 108.25 94) (end 102.45 94) (width 0.2) (layer F.Cu) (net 11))
 (segment (start 102.45 94) (end 99.25 97.2) (width 0.2) (layer F.Cu) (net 11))
 (segment (start 108.25 94.4) (end 103.65 94.4) (width 0.2) (layer F.Cu) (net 11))
 (segment (start 103.65 94.4) (end 99.25 98.8) (width 0.2) (layer F.Cu) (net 11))
 (segment (start 104.85 94.8) (end 99.25 100.4) (width 0.2) (layer F.Cu) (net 11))
 (segment (start 108.25 94.8) (end 104.85 94.8) (width 0.2) (layer F.Cu) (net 11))
 (segment (start 104.45 108.2) (end 99.25 103) (width 0.2) (layer F.Cu) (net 11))
 (segment (start 108.25 108.2) (end 104.45 108.2) (width 0.2) (layer F.Cu) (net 11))
 (segment (start 108.25 108.6) (end 103.25 108.6) (width 0.2) (layer F.Cu) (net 11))
 (segment (start 103.25 108.6) (end 99.25 104.6) (width 0.2) (layer F.Cu) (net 11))
 (segment (start 102.05 109) (end 99.25 106.2) (width 0.2) (layer F.Cu) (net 11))
 (segment (start 108.25 109) (end 102.05 109) (width 0.2) (layer F.Cu) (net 11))
 (segment (start 108.25 109.4) (end 100.85 109.4) (width 0.2) (layer F.Cu) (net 11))
 (segment (start 100.85 109.4) (end 99.25 107.8) (width 0.2) (layer F.Cu) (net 11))
 (segment (start 99.65 109.8) (end 99.25 109.4) (width 0.2) (layer F.Cu) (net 11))
 (segment (start 108.25 109.8) (end 99.65 109.8) (width 0.2) (layer F.Cu) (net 11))
 (segment (start 108.25 110.2) (end 100.05 110.2) (width 0.2) (layer F.Cu) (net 11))
 (segment (start 100.05 110.2) (end 99.25 111) (width 0.2) (layer F.Cu) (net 11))
 (segment (start 108.25 110.6) (end 101.25 110.6) (width 0.2) (layer F.Cu) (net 11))
 (segment (start 101.25 110.6) (end 99.25 112.6) (width 0.2) (layer F.Cu) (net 11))
 (segment (start 108.25 111) (end 102.45 111) (width 0.2) (layer F.Cu) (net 11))
 (segment (start 102.45 111) (end 99.25 114.2) (width 0.2) (layer F.Cu) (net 11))
 (segment (start 108.25 111.4) (end 103.65 111.4) (width 0.2) (layer F.Cu) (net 11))
 (segment (start 103.65 111.4) (end 99.25 115.8) (width 0.2) (layer F.Cu) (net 11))
 (segment (start 104.85 111.8) (end 99.25 117.4) (width 0.2) (layer F.Cu) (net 11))
 (segment (start 108.25 111.8) (end 104.85 111.8) (width 0.2) (layer F.Cu) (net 11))
 (segment (start 104.45 57.2) (end 99.25 52) (width 0.2) (layer F.Cu) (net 11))
 (segment (start 108.25 57.2) (end 104.45 57.2) (width 0.2) (layer F.Cu) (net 11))
 (segment (start 108.25 57.6) (end 103.25 57.6) (width 0.2) (layer F.Cu) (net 11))
 (segment (start 103.25 57.6) (end 99.25 53.6) (width 0.2) (layer F.Cu) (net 11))
 (segment (start 102.05 58) (end 99.25 55.2) (width 0.2) (layer F.Cu) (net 11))
 (segment (start 108.25 58) (end 102.05 58) (width 0.2) (layer F.Cu) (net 11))
 (segment (start 108.25 58.4) (end 100.85 58.4) (width 0.2) (layer F.Cu) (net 11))
 (segment (start 100.85 58.4) (end 99.25 56.8) (width 0.2) (layer F.Cu) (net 11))
 (segment (start 99.65 58.8) (end 99.25 58.4) (width 0.2) (layer F.Cu) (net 11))
 (segment (start 108.25 58.8) (end 99.65 58.8) (width 0.2) (layer F.Cu) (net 11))
 (segment (start 108.25 59.2) (end 100.05 59.2) (width 0.2) (layer F.Cu) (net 11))
 (segment (start 100.05 59.2) (end 99.25 60) (width 0.2) (layer F.Cu) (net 11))
 (segment (start 108.25 59.6) (end 101.25 59.6) (width 0.2) (layer F.Cu) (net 11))
 (segment (start 101.25 59.6) (end 99.25 61.6) (width 0.2) (layer F.Cu) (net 11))
 (segment (start 108.25 60) (end 102.45 60) (width 0.2) (layer F.Cu) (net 11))
 (segment (start 102.45 60) (end 99.25 63.2) (width 0.2) (layer F.Cu) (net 11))
 (segment (start 108.25 60.4) (end 103.65 60.4) (width 0.2) (layer F.Cu) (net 11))
 (segment (start 103.65 60.4) (end 99.25 64.8) (width 0.2) (layer F.Cu) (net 11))
 (segment (start 104.85 60.8) (end 99.25 66.4) (width 0.2) (layer F.Cu) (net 11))
 (segment (start 108.25 60.8) (end 104.85 60.8) (width 0.2) (layer F.Cu) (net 11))
 (segment (start 99.25 117.4) (end 99.25 115.8) (width 0.2) (layer F.Cu) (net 11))
 (segment (start 99.25 115.8) (end 99.25 114.2) (width 0.2) (layer F.Cu) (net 11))
 (segment (start 99.25 114.2) (end 99.25 112.6) (width 0.2) (layer F.Cu) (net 11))
 (segment (start 99.25 112.6) (end 99.25 111) (width 0.2) (layer F.Cu) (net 11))
 (segment (start 99.25 111) (end 99.25 109.4) (width 0.2) (layer F.Cu) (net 11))
 (segment (start 99.25 109.4) (end 99.25 107.8) (width 0.2) (layer F.Cu) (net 11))
 (segment (start 99.25 107.8) (end 99.25 106.2) (width 0.2) (layer F.Cu) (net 11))
 (segment (start 99.25 106.2) (end 99.25 104.6) (width 0.2) (layer F.Cu) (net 11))
 (segment (start 99.25 104.6) (end 99.25 103) (width 0.2) (layer F.Cu) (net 11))
 (segment (start 99.25 106) (end 99.25 100.4) (width 0.2) (layer F.Cu) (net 11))
 (segment (start 99.25 100.4) (end 99.25 98.8) (width 0.2) (layer F.Cu) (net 11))
 (segment (start 99.25 98.8) (end 99.25 97.2) (width 0.2) (layer F.Cu) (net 11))
 (segment (start 99.25 97.2) (end 99.25 95.6) (width 0.2) (layer F.Cu) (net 11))
 (segment (start 99.25 95.6) (end 99.25 94) (width 0.2) (layer F.Cu) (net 11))
 (segment (start 99.25 94) (end 99.25 92.4) (width 0.2) (layer F.Cu) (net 11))
 (segment (start 99.25 92.4) (end 99.25 90.8) (width 0.2) (layer F.Cu) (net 11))
 (segment (start 99.25 90.8) (end 99.25 89.2) (width 0.2) (layer F.Cu) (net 11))
 (segment (start 99.25 89.2) (end 99.25 87.6) (width 0.2) (layer F.Cu) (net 11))
 (segment (start 99.25 87.6) (end 99.25 86) (width 0.2) (layer F.Cu) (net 11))
 (segment (start 99.25 89) (end 99.25 83.4) (width 0.2) (layer F.Cu) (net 11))
 (segment (start 99.25 83.4) (end 99.25 81.8) (width 0.2) (layer F.Cu) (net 11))
 (segment (start 99.25 81.8) (end 99.25 80.2) (width 0.2) (layer F.Cu) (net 11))
 (segment (start 99.25 80.2) (end 99.25 78.6) (width 0.2) (layer F.Cu) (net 11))
 (segment (start 99.25 78.6) (end 99.25 77) (width 0.2) (layer F.Cu) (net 11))
 (segment (start 99.25 77) (end 99.25 75.4) (width 0.2) (layer F.Cu) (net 11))
 (segment (start 99.25 75.4) (end 99.25 73.8) (width 0.2) (layer F.Cu) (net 11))
 (segment (start 99.25 73.8) (end 99.25 72.2) (width 0.2) (layer F.Cu) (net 11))
 (segment (start 99.25 72.2) (end 99.25 70.6) (width 0.2) (layer F.Cu) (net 11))
 (segment (start 99.25 70.6) (end 99.25 69) (width 0.2) (layer F.Cu) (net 11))
 (segment (start 99.25 69) (end 99.25 63.4) (width 0.2) (layer F.Cu) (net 11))
 (segment (start 99.25 66.4) (end 99.25 64.8) (width 0.2) (layer F.Cu) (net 11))
 (segment (start 99.25 64.8) (end 99.25 63.2) (width 0.2) (layer F.Cu) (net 11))
 (segment (start 99.25 63.2) (end 99.25 61.6) (width 0.2) (layer F.Cu) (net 11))
 (segment (start 99.25 61.6) (end 99.25 60) (width 0.2) (layer F.Cu) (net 11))
 (segment (start 99.25 60) (end 99.25 58.4) (width 0.2) (layer F.Cu) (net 11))
 (segment (start 99.25 58.4) (end 99.25 56.8) (width 0.2) (layer F.Cu) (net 11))
 (segment (start 99.25 56.8) (end 99.25 55.2) (width 0.2) (layer F.Cu) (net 11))
 (segment (start 99.25 55.2) (end 99.25 53.6) (width 0.2) (layer F.Cu) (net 11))
 (segment (start 99.25 53.6) (end 99.25 52) (width 0.2) (layer F.Cu) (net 11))
 (segment (start 99.25 52) (end 99.25 50.25) (width 0.2) (layer F.Cu) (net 11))
 (segment (start 99.25 50.25) (end 100 49.5) (width 0.2) (layer F.Cu) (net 11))
 (segment (start 110.25 58.4) (end 117.65 58.4) (width 0.2) (layer F.Cu) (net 2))
 (segment (start 117.65 58.4) (end 119.25 56.8) (width 0.2) (layer F.Cu) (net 2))
 (segment (start 118.45 59.2) (end 119.25 60) (width 0.2) (layer F.Cu) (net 3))
 (segment (start 110.25 59.2) (end 118.45 59.2) (width 0.2) (layer F.Cu) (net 3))
 (segment (start 110.25 60.8) (end 113.65 60.8) (width 0.2) (layer F.Cu) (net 4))
 (segment (start 113.65 60.8) (end 119.25 66.4) (width 0.2) (layer F.Cu) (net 4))
 (segment (start 116.05 60) (end 119.25 63.2) (width 0.2) (layer F.Cu) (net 5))
 (segment (start 110.25 60) (end 116.05 60) (width 0.2) (layer F.Cu) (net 5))
 (segment (start 110.25 57.6) (end 115.25 57.6) (width 0.2) (layer F.Cu) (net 6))
 (segment (start 115.25 57.6) (end 119.25 53.6) (width 0.2) (layer F.Cu) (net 6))
 (segment (start 110.25 75.4) (end 117.65 75.4) (width 0.2) (layer F.Cu) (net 33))
 (segment (start 117.65 75.4) (end 119.25 73.8) (width 0.2) (layer F.Cu) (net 33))
 (segment (start 118.45 76.2) (end 119.25 77) (width 0.2) (layer F.Cu) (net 34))
 (segment (start 110.25 76.2) (end 118.45 76.2) (width 0.2) (layer F.Cu) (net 34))
 (segment (start 110.25 77.8) (end 113.65 77.8) (width 0.2) (layer F.Cu) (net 35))
 (segment (start 113.65 77.8) (end 119.25 83.4) (width 0.2) (layer F.Cu) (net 35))
 (segment (start 116.05 77) (end 119.25 80.2) (width 0.2) (layer F.Cu) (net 36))
 (segment (start 110.25 77) (end 116.05 77) (width 0.2) (layer F.Cu) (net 36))
 (segment (start 110.25 74.6) (end 115.25 74.6) (width 0.2) (layer F.Cu) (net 37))
 (segment (start 115.25 74.6) (end 119.25 70.6) (width 0.2) (layer F.Cu) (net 37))
 (segment (start 110.25 92.4) (end 117.65 92.4) (width 0.2) (layer F.Cu) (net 23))
 (segment (start 117.65 92.4) (end 119.25 90.8) (width 0.2) (layer F.Cu) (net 23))
 (segment (start 118.45 93.2) (end 119.25 94) (width 0.2) (layer F.Cu) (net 24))
 (segment (start 110.25 93.2) (end 118.45 93.2) (width 0.2) (layer F.Cu) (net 24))
 (segment (start 110.25 94.8) (end 113.65 94.8) (width 0.2) (layer F.Cu) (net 25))
 (segment (start 113.65 94.8) (end 119.25 100.4) (width 0.2) (layer F.Cu) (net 25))
 (segment (start 116.05 94) (end 119.25 97.2) (width 0.2) (layer F.Cu) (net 26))
 (segment (start 110.25 94) (end 116.05 94) (width 0.2) (layer F.Cu) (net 26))
 (segment (start 110.25 91.6) (end 115.25 91.6) (width 0.2) (layer F.Cu) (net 27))
 (segment (start 115.25 91.6) (end 119.25 87.6) (width 0.2) (layer F.Cu) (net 27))
 (segment (start 110.25 109.4) (end 117.65 109.4) (width 0.2) (layer F.Cu) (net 13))
 (segment (start 117.65 109.4) (end 119.25 107.8) (width 0.2) (layer F.Cu) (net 13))
 (segment (start 118.45 110.2) (end 119.25 111) (width 0.2) (layer F.Cu) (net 14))
 (segment (start 110.25 110.2) (end 118.45 110.2) (width 0.2) (layer F.Cu) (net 14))
 (segment (start 110.25 111.8) (end 113.65 111.8) (width 0.2) (layer F.Cu) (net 15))
 (segment (start 113.65 111.8) (end 119.25 117.4) (width 0.2) (layer F.Cu) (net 15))
 (segment (start 116.05 111) (end 119.25 114.2) (width 0.2) (layer F.Cu) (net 16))
 (segment (start 110.25 111) (end 116.05 111) (width 0.2) (layer F.Cu) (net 16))
 (segment (start 110.25 108.6) (end 115.25 108.6) (width 0.2) (layer F.Cu) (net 17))
 (segment (start 115.25 108.6) (end 119.25 104.6) (width 0.2) (layer F.Cu) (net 17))
 (segment (start 118.85 58.8) (end 119.25 58.4) (width 0.2) (layer F.Cu) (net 1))
 (segment (start 110.25 58.8) (end 118.85 58.8) (width 0.2) (layer F.Cu) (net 1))
 (segment (start 114.05 57.2) (end 119.25 52) (width 0.2) (layer F.Cu) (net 9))
 (segment (start 110.25 57.2) (end 114.05 57.2) (width 0.2) (layer F.Cu) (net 9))
 (segment (start 110.25 59.6) (end 117.25 59.6) (width 0.2) (layer F.Cu) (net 7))
 (segment (start 117.25 59.6) (end 119.25 61.6) (width 0.2) (layer F.Cu) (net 7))
 (segment (start 114.85 60.4) (end 119.25 64.8) (width 0.2) (layer F.Cu) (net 10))
 (segment (start 110.25 60.4) (end 114.85 60.4) (width 0.2) (layer F.Cu) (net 10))
 (segment (start 116.45 58) (end 119.25 55.2) (width 0.2) (layer F.Cu) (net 8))
 (segment (start 110.25 58) (end 116.45 58) (width 0.2) (layer F.Cu) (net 8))
 (segment (start 118.85 75.8) (end 119.25 75.4) (width 0.2) (layer F.Cu) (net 32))
 (segment (start 110.25 75.8) (end 118.85 75.8) (width 0.2) (layer F.Cu) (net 32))
 (segment (start 110.25 76.6) (end 117.25 76.6) (width 0.2) (layer F.Cu) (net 38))
 (segment (start 117.25 76.6) (end 119.25 78.6) (width 0.2) (layer F.Cu) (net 38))
 (segment (start 116.45 75) (end 119.25 72.2) (width 0.2) (layer F.Cu) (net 39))
 (segment (start 110.25 75) (end 116.45 75) (width 0.2) (layer F.Cu) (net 39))
 (segment (start 114.05 74.2) (end 119.25 69) (width 0.2) (layer F.Cu) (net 40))
 (segment (start 110.25 74.2) (end 114.05 74.2) (width 0.2) (layer F.Cu) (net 40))
 (segment (start 114.85 77.4) (end 119.25 81.8) (width 0.2) (layer F.Cu) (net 41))
 (segment (start 110.25 77.4) (end 114.85 77.4) (width 0.2) (layer F.Cu) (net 41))
 (segment (start 118.85 92.8) (end 119.25 92.4) (width 0.2) (layer F.Cu) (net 22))
 (segment (start 110.25 92.8) (end 118.85 92.8) (width 0.2) (layer F.Cu) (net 22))
 (segment (start 114.05 91.2) (end 119.25 86) (width 0.2) (layer F.Cu) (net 30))
 (segment (start 110.25 91.2) (end 114.05 91.2) (width 0.2) (layer F.Cu) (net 30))
 (segment (start 110.25 93.6) (end 117.25 93.6) (width 0.2) (layer F.Cu) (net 28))
 (segment (start 117.25 93.6) (end 119.25 95.6) (width 0.2) (layer F.Cu) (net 28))
 (segment (start 114.85 94.4) (end 119.25 98.8) (width 0.2) (layer F.Cu) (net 31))
 (segment (start 110.25 94.4) (end 114.85 94.4) (width 0.2) (layer F.Cu) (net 31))
 (segment (start 116.45 92) (end 119.25 89.2) (width 0.2) (layer F.Cu) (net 29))
 (segment (start 110.25 92) (end 116.45 92) (width 0.2) (layer F.Cu) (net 29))
 (segment (start 118.85 109.8) (end 119.25 109.4) (width 0.2) (layer F.Cu) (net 12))
 (segment (start 110.25 109.8) (end 118.85 109.8) (width 0.2) (layer F.Cu) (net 12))
 (segment (start 110.25 110.6) (end 117.25 110.6) (width 0.2) (layer F.Cu) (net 18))
 (segment (start 117.25 110.6) (end 119.25 112.6) (width 0.2) (layer F.Cu) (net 18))
 (segment (start 116.45 109) (end 119.25 106.2) (width 0.2) (layer F.Cu) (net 19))
 (segment (start 110.25 109) (end 116.45 109) (width 0.2) (layer F.Cu) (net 19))
 (segment (start 114.05 108.2) (end 119.25 103) (width 0.2) (layer F.Cu) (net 20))
 (segment (start 110.25 108.2) (end 114.05 108.2) (width 0.2) (layer F.Cu) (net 20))
 (segment (start 114.85 111.4) (end 119.25 115.8) (width 0.2) (layer F.Cu) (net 21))
 (segment (start 110.25 111.4) (end 114.85 111.4) (width 0.2) (layer F.Cu) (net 21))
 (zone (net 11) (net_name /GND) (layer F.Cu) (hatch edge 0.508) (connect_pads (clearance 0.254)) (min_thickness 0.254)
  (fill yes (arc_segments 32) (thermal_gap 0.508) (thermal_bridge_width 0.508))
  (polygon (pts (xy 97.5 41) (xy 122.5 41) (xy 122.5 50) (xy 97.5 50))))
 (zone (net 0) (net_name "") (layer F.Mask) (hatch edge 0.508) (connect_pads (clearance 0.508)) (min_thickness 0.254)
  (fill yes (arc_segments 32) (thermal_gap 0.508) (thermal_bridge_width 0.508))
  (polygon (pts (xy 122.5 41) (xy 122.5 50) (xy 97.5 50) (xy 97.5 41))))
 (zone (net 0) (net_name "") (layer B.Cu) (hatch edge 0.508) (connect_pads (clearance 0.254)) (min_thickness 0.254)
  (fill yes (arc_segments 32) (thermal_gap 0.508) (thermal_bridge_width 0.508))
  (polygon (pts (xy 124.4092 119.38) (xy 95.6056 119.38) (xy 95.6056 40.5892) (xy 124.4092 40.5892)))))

